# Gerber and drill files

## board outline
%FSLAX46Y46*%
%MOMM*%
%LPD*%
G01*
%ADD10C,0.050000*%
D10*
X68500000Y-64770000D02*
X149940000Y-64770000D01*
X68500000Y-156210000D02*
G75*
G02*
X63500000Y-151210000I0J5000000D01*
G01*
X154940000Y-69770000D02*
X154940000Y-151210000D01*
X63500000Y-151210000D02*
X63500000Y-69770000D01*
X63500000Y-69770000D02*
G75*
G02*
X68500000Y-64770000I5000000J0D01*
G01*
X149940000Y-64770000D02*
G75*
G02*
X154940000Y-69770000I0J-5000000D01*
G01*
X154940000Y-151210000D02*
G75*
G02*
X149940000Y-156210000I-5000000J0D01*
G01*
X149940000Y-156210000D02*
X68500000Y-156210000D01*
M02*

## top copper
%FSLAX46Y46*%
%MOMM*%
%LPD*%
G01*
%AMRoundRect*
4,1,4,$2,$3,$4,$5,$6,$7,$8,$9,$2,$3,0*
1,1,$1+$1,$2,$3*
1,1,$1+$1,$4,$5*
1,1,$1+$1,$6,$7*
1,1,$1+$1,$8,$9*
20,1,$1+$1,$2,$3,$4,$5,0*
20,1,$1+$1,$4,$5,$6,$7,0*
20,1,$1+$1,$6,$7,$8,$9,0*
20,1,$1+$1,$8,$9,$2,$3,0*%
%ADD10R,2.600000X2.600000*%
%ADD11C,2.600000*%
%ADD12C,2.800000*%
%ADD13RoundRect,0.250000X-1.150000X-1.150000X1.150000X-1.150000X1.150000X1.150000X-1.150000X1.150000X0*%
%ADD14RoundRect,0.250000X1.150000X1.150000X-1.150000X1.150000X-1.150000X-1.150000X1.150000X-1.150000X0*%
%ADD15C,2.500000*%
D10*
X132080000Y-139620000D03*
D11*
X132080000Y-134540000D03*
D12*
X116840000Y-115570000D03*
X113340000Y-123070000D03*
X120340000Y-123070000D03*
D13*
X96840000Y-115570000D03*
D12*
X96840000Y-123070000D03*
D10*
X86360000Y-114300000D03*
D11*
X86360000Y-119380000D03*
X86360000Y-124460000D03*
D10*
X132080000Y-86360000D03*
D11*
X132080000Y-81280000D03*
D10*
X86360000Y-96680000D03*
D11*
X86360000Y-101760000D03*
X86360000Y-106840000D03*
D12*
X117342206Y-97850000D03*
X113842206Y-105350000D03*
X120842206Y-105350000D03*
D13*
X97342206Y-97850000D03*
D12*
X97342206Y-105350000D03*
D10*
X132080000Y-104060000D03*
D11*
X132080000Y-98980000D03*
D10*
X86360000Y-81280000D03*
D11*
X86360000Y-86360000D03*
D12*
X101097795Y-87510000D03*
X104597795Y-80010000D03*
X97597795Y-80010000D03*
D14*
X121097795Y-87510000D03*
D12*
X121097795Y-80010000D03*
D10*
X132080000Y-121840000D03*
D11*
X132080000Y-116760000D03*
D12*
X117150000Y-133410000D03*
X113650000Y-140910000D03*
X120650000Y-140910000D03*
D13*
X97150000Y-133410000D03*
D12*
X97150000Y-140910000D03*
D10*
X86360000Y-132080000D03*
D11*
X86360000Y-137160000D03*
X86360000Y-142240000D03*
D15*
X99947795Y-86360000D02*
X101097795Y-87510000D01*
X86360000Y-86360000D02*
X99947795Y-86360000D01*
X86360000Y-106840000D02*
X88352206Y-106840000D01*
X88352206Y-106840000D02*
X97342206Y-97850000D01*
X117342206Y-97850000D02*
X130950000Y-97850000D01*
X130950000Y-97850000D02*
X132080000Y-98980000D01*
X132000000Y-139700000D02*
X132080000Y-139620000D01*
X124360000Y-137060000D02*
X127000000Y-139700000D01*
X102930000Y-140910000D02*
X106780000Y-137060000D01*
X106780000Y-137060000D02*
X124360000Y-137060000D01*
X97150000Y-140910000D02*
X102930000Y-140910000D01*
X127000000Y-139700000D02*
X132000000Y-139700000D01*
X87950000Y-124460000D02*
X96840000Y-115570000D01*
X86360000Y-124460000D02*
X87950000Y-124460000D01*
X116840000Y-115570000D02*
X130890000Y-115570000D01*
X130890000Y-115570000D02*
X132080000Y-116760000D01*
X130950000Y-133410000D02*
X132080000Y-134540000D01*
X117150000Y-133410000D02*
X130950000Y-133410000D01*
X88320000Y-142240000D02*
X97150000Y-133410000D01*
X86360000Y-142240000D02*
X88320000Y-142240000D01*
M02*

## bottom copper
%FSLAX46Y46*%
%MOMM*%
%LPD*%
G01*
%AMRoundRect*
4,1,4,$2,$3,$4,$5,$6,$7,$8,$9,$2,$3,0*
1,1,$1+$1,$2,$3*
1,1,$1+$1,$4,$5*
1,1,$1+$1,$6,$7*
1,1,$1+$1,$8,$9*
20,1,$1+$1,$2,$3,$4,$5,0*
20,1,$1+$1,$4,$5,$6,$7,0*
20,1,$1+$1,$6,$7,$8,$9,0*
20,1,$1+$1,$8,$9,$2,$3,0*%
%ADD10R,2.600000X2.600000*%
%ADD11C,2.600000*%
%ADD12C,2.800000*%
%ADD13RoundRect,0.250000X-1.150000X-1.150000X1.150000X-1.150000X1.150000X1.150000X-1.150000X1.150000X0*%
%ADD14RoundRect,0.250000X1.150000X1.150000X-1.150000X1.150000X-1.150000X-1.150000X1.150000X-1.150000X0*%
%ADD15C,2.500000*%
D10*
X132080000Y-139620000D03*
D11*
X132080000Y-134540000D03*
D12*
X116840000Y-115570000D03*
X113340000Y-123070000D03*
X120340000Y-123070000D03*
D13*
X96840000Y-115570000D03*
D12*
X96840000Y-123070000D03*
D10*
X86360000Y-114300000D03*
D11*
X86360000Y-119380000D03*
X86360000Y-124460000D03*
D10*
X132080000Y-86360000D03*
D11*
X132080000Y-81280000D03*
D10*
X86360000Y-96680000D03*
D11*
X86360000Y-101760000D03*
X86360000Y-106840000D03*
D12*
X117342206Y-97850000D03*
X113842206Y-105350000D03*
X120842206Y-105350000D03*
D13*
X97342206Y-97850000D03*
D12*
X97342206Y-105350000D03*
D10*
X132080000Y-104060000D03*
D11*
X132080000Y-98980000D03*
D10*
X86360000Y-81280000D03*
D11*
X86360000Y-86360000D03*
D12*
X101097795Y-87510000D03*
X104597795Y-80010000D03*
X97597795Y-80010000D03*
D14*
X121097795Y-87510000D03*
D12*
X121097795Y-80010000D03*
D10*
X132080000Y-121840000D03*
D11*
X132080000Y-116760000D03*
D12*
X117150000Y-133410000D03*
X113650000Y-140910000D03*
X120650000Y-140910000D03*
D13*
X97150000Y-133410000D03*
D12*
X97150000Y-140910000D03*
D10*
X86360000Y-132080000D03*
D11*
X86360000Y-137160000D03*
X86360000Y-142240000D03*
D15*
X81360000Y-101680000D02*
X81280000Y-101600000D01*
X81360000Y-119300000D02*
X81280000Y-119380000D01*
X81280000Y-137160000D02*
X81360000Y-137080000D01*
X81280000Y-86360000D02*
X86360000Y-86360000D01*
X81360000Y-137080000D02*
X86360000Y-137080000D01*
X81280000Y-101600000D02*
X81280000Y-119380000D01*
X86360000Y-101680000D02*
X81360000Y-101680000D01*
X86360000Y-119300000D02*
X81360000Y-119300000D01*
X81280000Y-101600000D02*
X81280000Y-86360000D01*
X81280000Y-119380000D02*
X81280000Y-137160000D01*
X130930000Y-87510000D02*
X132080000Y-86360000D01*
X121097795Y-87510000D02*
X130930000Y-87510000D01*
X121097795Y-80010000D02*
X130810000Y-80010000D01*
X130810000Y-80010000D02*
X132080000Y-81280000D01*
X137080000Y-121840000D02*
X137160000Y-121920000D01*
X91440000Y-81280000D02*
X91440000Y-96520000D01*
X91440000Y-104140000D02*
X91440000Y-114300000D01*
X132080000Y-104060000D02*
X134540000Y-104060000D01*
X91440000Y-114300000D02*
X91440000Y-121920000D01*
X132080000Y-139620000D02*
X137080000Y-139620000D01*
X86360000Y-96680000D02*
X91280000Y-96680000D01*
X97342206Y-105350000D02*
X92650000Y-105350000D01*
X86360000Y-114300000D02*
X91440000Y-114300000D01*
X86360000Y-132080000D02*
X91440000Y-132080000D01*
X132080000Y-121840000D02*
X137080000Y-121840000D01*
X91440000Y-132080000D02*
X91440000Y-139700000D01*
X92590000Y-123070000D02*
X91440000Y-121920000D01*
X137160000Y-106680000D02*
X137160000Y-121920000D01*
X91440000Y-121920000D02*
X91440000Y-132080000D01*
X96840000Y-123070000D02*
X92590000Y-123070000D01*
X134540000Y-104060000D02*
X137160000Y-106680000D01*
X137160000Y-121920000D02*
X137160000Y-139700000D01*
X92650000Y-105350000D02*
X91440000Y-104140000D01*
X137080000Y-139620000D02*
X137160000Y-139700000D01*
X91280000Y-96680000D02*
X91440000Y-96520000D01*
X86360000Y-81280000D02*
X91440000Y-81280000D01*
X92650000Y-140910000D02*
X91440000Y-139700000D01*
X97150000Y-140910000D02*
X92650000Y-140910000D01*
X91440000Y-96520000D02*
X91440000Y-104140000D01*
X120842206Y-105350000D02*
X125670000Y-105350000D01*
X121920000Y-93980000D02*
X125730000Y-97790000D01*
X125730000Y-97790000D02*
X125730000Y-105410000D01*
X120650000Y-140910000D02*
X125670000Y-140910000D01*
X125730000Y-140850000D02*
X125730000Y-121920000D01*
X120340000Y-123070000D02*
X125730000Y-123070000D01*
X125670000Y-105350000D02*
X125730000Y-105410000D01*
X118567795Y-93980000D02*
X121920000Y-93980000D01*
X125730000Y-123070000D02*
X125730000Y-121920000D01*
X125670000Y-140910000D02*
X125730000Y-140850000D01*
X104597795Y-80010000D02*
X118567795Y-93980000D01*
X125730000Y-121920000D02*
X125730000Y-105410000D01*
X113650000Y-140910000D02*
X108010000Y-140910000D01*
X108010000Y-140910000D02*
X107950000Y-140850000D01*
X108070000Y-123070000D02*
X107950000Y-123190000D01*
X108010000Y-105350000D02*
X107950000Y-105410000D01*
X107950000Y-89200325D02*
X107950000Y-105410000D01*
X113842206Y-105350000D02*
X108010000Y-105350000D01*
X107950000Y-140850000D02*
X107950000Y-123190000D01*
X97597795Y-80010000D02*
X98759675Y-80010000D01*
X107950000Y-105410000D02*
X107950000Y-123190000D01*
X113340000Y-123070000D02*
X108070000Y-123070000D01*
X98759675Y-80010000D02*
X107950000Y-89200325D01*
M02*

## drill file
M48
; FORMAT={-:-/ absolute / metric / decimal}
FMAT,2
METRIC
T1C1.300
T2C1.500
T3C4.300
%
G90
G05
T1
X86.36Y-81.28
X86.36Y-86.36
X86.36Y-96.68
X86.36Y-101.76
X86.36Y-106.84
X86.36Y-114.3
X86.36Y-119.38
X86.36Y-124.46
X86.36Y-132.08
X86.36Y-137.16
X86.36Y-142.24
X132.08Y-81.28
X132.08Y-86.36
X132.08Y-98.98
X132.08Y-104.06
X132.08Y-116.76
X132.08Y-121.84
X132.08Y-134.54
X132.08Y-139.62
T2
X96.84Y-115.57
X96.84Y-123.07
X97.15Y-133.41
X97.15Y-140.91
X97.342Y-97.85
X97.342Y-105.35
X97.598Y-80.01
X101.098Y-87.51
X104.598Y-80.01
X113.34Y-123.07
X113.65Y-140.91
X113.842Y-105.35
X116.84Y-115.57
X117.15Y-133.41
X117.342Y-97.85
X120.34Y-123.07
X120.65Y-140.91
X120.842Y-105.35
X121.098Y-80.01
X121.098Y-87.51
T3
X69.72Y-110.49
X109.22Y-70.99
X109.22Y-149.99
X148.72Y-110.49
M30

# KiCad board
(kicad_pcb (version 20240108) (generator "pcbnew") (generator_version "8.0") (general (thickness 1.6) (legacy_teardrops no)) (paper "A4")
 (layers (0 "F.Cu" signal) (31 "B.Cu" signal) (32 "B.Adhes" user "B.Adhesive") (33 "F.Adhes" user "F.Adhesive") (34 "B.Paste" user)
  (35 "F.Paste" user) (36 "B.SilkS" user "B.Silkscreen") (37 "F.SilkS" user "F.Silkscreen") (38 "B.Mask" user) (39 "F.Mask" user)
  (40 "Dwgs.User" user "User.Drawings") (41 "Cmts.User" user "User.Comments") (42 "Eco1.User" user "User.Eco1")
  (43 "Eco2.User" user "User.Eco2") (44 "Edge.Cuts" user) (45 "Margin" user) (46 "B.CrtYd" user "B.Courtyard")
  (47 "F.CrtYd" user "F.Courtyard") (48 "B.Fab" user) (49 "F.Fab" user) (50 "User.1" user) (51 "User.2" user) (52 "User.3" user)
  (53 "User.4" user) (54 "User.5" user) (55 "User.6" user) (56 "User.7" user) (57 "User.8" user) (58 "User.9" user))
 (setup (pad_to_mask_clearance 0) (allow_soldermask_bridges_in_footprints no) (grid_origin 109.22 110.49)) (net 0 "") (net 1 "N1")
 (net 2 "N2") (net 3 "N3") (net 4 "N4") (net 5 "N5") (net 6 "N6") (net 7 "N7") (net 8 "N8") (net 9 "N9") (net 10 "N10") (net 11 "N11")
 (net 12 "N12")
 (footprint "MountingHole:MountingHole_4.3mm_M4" (layer "F.Cu") (at 109.22 149.99)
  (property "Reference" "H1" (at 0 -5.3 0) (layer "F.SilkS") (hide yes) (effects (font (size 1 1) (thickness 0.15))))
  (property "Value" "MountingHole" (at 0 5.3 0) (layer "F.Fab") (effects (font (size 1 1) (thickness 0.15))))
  (pad "" np_thru_hole circle (at 0 0) (size 4.3 4.3) (drill 4.3) (layers "*.Cu" "*.Mask")))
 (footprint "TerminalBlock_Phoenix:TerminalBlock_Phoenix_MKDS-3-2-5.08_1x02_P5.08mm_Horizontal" (layer "F.Cu") (at 132.08 139.62 90)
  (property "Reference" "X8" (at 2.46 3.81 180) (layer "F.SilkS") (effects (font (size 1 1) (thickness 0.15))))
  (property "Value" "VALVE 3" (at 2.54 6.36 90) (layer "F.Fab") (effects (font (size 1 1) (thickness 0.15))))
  (pad "1" thru_hole rect (at 0 0 90) (size 2.6 2.6) (drill 1.3) (layers "*.Cu" "*.Mask") (remove_unused_layers no) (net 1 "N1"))
  (pad "2" thru_hole circle (at 5.08 0 90) (size 2.6 2.6) (drill 1.3) (layers "*.Cu" "*.Mask") (remove_unused_layers no) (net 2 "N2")))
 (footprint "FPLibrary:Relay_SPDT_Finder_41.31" (layer "F.Cu") (at 96.84 115.57)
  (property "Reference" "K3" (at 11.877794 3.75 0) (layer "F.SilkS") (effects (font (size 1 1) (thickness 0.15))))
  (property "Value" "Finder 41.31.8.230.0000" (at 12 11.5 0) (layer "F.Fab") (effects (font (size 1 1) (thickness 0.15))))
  (pad "11" thru_hole circle (at 20 0) (size 2.8 2.8) (drill 1.5) (layers "*.Cu" "*.Mask") (remove_unused_layers no) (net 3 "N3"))
  (pad "12" thru_hole circle (at 16.5 7.5) (size 2.8 2.8) (drill 1.5) (layers "*.Cu" "*.Mask") (remove_unused_layers no) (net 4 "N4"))
  (pad "14" thru_hole circle (at 23.5 7.5) (size 2.8 2.8) (drill 1.5) (layers "*.Cu" "*.Mask") (remove_unused_layers no) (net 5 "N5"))
  (pad "A1" thru_hole roundrect (at 0 0) (size 2.8 2.8) (drill 1.5) (layers "*.Cu" "*.Mask") (remove_unused_layers no)
   (roundrect_rratio 0.08928571429) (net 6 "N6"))
  (pad "A2" thru_hole circle (at 0 7.5) (size 2.8 2.8) (drill 1.5) (layers "*.Cu" "*.Mask") (remove_unused_layers no) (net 1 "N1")))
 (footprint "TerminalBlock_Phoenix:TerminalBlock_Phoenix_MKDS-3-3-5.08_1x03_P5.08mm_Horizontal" (layer "F.Cu") (at 86.36 114.3 -90)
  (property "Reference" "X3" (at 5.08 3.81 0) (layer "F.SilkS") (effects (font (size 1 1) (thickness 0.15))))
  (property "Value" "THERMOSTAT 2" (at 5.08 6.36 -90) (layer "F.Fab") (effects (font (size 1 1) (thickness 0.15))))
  (pad "1" thru_hole rect (at 0 0 270) (size 2.6 2.6) (drill 1.3) (layers "*.Cu" "*.Mask") (remove_unused_layers no) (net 1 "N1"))
  (pad "2" thru_hole circle (at 5.08 0 270) (size 2.6 2.6) (drill 1.3) (layers "*.Cu" "*.Mask") (remove_unused_layers no) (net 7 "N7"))
  (pad "3" thru_hole circle (at 10.16 0 270) (size 2.6 2.6) (drill 1.3) (layers "*.Cu" "*.Mask") (remove_unused_layers no) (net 6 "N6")))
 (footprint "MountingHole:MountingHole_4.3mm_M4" (layer "F.Cu") (at 69.72 110.49)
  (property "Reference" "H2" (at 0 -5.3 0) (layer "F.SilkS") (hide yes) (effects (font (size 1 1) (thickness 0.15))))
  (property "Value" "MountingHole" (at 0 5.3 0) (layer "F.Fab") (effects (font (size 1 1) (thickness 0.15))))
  (pad "" np_thru_hole circle (at 0 0) (size 4.3 4.3) (drill 4.3) (layers "*.Cu" "*.Mask")))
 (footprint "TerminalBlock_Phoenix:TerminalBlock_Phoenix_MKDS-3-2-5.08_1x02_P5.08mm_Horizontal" (layer "F.Cu") (at 132.08 86.36 90)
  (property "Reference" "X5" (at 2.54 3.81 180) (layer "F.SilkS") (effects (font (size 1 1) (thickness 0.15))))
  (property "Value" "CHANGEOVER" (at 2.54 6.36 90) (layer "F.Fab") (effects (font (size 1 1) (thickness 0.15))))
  (pad "1" thru_hole rect (at 0 0 90) (size 2.6 2.6) (drill 1.3) (layers "*.Cu" "*.Mask") (remove_unused_layers no) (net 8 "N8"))
  (pad "2" thru_hole circle (at 5.08 0 90) (size 2.6 2.6) (drill 1.3) (layers "*.Cu" "*.Mask") (remove_unused_layers no) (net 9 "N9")))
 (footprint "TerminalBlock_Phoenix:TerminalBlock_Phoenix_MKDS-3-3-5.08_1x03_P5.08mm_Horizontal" (layer "F.Cu") (at 86.36 96.68 -90)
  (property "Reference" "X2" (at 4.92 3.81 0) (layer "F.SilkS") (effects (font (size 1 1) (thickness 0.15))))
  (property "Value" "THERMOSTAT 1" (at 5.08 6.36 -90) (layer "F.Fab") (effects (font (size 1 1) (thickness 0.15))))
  (pad "1" thru_hole rect (at 0 0 270) (size 2.6 2.6) (drill 1.3) (layers "*.Cu" "*.Mask") (remove_unused_layers no) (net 1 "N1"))
  (pad "2" thru_hole circle (at 5.08 0 270) (size 2.6 2.6) (drill 1.3) (layers "*.Cu" "*.Mask") (remove_unused_layers no) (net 7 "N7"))
  (pad "3" thru_hole circle (at 10.16 0 270) (size 2.6 2.6) (drill 1.3) (layers "*.Cu" "*.Mask") (remove_unused_layers no) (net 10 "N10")))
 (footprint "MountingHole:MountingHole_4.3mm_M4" (layer "F.Cu") (at 109.22 70.99)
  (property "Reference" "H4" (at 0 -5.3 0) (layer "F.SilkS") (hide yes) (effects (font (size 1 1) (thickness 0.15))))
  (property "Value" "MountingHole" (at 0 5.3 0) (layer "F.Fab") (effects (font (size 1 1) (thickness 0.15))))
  (pad "" np_thru_hole circle (at 0 0) (size 4.3 4.3) (drill 4.3) (layers "*.Cu" "*.Mask")))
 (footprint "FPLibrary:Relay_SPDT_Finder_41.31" (layer "F.Cu") (at 97.342206 97.85)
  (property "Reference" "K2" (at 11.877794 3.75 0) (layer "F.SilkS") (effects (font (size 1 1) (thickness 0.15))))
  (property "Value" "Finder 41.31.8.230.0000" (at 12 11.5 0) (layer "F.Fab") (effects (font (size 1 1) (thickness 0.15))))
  (pad "11" thru_hole circle (at 20 0) (size 2.8 2.8) (drill 1.5) (layers "*.Cu" "*.Mask") (remove_unused_layers no) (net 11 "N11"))
  (pad "12" thru_hole circle (at 16.5 7.5) (size 2.8 2.8) (drill 1.5) (layers "*.Cu" "*.Mask") (remove_unused_layers no) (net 4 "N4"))
  (pad "14" thru_hole circle (at 23.5 7.5) (size 2.8 2.8) (drill 1.5) (layers "*.Cu" "*.Mask") (remove_unused_layers no) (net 5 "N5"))
  (pad "A1" thru_hole roundrect (at 0 0) (size 2.8 2.8) (drill 1.5) (layers "*.Cu" "*.Mask") (remove_unused_layers no)
   (roundrect_rratio 0.08928571429) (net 10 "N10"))
  (pad "A2" thru_hole circle (at 0 7.5) (size 2.8 2.8) (drill 1.5) (layers "*.Cu" "*.Mask") (remove_unused_layers no) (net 1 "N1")))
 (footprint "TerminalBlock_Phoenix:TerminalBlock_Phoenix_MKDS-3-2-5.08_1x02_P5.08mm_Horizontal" (layer "F.Cu") (at 132.08 104.06 90)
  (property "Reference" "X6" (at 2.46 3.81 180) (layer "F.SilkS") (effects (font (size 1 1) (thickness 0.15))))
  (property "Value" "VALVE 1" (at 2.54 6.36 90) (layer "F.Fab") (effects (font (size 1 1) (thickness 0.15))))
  (pad "1" thru_hole rect (at 0 0 90) (size 2.6 2.6) (drill 1.3) (layers "*.Cu" "*.Mask") (remove_unused_layers no) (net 1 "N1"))
  (pad "2" thru_hole circle (at 5.08 0 90) (size 2.6 2.6) (drill 1.3) (layers "*.Cu" "*.Mask") (remove_unused_layers no) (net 11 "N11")))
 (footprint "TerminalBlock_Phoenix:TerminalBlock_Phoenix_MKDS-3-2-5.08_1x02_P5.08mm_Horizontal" (layer "F.Cu") (at 86.36 81.28 -90)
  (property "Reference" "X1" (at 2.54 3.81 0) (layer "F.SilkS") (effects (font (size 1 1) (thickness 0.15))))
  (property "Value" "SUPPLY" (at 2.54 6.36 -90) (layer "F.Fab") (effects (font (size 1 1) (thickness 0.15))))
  (pad "1" thru_hole rect (at 0 0 270) (size 2.6 2.6) (drill 1.3) (layers "*.Cu" "*.Mask") (remove_unused_layers no) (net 1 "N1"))
  (pad "2" thru_hole circle (at 5.08 0 270) (size 2.6 2.6) (drill 1.3) (layers "*.Cu" "*.Mask") (remove_unused_layers no) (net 7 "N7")))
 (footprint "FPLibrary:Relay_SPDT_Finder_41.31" (layer "F.Cu") (at 121.097795 87.51 180)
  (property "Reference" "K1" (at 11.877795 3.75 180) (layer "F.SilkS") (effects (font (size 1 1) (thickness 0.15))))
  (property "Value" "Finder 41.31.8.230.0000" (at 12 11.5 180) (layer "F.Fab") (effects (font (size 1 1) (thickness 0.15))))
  (pad "11" thru_hole circle (at 20 0 180) (size 2.8 2.8) (drill 1.5) (layers "*.Cu" "*.Mask") (remove_unused_layers no) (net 7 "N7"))
  (pad "12" thru_hole circle (at 16.5 7.5 180) (size 2.8 2.8) (drill 1.5) (layers "*.Cu" "*.Mask") (remove_unused_layers no) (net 5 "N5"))
  (pad "14" thru_hole circle (at 23.5 7.5 180) (size 2.8 2.8) (drill 1.5) (layers "*.Cu" "*.Mask") (remove_unused_layers no) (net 4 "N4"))
  (pad "A1" thru_hole roundrect (at 0 0 180) (size 2.8 2.8) (drill 1.5) (layers "*.Cu" "*.Mask") (remove_unused_layers no)
   (roundrect_rratio 0.08928571429) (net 8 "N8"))
  (pad "A2" thru_hole circle (at 0 7.5 180) (size 2.8 2.8) (drill 1.5) (layers "*.Cu" "*.Mask") (remove_unused_layers no) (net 9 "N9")))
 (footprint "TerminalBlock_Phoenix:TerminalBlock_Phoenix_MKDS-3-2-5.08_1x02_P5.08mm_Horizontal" (layer "F.Cu") (at 132.08 121.84 90)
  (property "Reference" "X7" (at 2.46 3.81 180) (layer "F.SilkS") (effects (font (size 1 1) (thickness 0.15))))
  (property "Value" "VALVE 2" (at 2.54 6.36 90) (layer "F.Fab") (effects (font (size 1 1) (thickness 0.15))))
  (pad "1" thru_hole rect (at 0 0 90) (size 2.6 2.6) (drill 1.3) (layers "*.Cu" "*.Mask") (remove_unused_layers no) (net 1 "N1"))
  (pad "2" thru_hole circle (at 5.08 0 90) (size 2.6 2.6) (drill 1.3) (layers "*.Cu" "*.Mask") (remove_unused_layers no) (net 3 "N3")))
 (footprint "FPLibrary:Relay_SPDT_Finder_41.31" (layer "F.Cu") (at 97.15 133.41)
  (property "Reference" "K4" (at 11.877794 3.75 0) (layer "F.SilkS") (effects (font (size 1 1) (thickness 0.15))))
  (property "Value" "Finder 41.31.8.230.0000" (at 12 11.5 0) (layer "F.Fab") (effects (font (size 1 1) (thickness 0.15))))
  (pad "11" thru_hole circle (at 20 0) (size 2.8 2.8) (drill 1.5) (layers "*.Cu" "*.Mask") (remove_unused_layers no) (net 2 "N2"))
  (pad "12" thru_hole circle (at 16.5 7.5) (size 2.8 2.8) (drill 1.5) (layers "*.Cu" "*.Mask") (remove_unused_layers no) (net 4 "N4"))
  (pad "14" thru_hole circle (at 23.5 7.5) (size 2.8 2.8) (drill 1.5) (layers "*.Cu" "*.Mask") (remove_unused_layers no) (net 5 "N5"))
  (pad "A1" thru_hole roundrect (at 0 0) (size 2.8 2.8) (drill 1.5) (layers "*.Cu" "*.Mask") (remove_unused_layers no)
   (roundrect_rratio 0.08928571429) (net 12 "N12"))
  (pad "A2" thru_hole circle (at 0 7.5) (size 2.8 2.8) (drill 1.5) (layers "*.Cu" "*.Mask") (remove_unused_layers no) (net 1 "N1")))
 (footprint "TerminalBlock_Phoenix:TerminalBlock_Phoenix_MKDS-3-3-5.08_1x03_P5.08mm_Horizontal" (layer "F.Cu") (at 86.36 132.08 -90)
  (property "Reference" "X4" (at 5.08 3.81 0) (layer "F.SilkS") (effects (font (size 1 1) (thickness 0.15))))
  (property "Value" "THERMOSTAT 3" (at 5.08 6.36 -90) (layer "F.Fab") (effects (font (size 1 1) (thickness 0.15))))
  (pad "1" thru_hole rect (at 0 0 270) (size 2.6 2.6) (drill 1.3) (layers "*.Cu" "*.Mask") (remove_unused_layers no) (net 1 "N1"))
  (pad "2" thru_hole circle (at 5.08 0 270) (size 2.6 2.6) (drill 1.3) (layers "*.Cu" "*.Mask") (remove_unused_layers no) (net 7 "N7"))
  (pad "3" thru_hole circle (at 10.16 0 270) (size 2.6 2.6) (drill 1.3) (layers "*.Cu" "*.Mask") (remove_unused_layers no) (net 12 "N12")))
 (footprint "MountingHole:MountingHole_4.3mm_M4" (layer "F.Cu") (at 148.72 110.49)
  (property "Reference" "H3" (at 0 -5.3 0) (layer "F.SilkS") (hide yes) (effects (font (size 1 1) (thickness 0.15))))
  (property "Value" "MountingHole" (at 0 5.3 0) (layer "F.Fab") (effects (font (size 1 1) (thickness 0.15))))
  (pad "" np_thru_hole circle (at 0 0) (size 4.3 4.3) (drill 4.3) (layers "*.Cu" "*.Mask")))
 (gr_line (start 68.5 64.77) (end 149.94 64.77) (stroke (width 0.05) (type default)) (layer "Edge.Cuts"))
 (gr_arc (start 68.5 156.21) (mid 64.964466 154.745534) (end 63.5 151.21) (stroke (width 0.05) (type default)) (layer "Edge.Cuts"))
 (gr_line (start 154.94 69.77) (end 154.94 151.21) (stroke (width 0.05) (type default)) (layer "Edge.Cuts"))
 (gr_line (start 63.5 151.21) (end 63.5 69.77) (stroke (width 0.05) (type default)) (layer "Edge.Cuts"))
 (gr_arc (start 63.5 69.77) (mid 64.964466 66.234466) (end 68.5 64.77) (stroke (width 0.05) (type default)) (layer "Edge.Cuts"))
 (gr_arc (start 149.94 64.77) (mid 153.475534 66.234466) (end 154.94 69.77) (stroke (width 0.05) (type default)) (layer "Edge.Cuts"))
 (gr_arc (start 154.94 151.21) (mid 153.475534 154.745534) (end 149.94 156.21) (stroke (width 0.05) (type default)) (layer "Edge.Cuts"))
 (gr_line (start 149.94 156.21) (end 68.5 156.21) (stroke (width 0.05) (type default)) (layer "Edge.Cuts"))
 (segment (start 99.947795 86.36) (end 101.097795 87.51) (width 2.5) (layer "F.Cu") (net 7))
 (segment (start 86.36 86.36) (end 99.947795 86.36) (width 2.5) (layer "F.Cu") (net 7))
 (segment (start 81.36 101.68) (end 81.28 101.6) (width 2.5) (layer "B.Cu") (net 7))
 (segment (start 81.36 119.3) (end 81.28 119.38) (width 2.5) (layer "B.Cu") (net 7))
 (segment (start 81.28 137.16) (end 81.36 137.08) (width 2.5) (layer "B.Cu") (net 7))
 (segment (start 81.28 86.36) (end 86.36 86.36) (width 2.5) (layer "B.Cu") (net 7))
 (segment (start 81.36 137.08) (end 86.36 137.08) (width 2.5) (layer "B.Cu") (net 7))
 (segment (start 81.28 101.6) (end 81.28 119.38) (width 2.5) (layer "B.Cu") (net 7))
 (segment (start 86.36 101.68) (end 81.36 101.68) (width 2.5) (layer "B.Cu") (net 7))
 (segment (start 86.36 119.3) (end 81.36 119.3) (width 2.5) (layer "B.Cu") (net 7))
 (segment (start 81.28 101.6) (end 81.28 86.36) (width 2.5) (layer "B.Cu") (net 7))
 (segment (start 81.28 119.38) (end 81.28 137.16) (width 2.5) (layer "B.Cu") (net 7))
 (segment (start 130.93 87.51) (end 132.08 86.36) (width 2.5) (layer "B.Cu") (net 8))
 (segment (start 121.097795 87.51) (end 130.93 87.51) (width 2.5) (layer "B.Cu") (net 8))
 (segment (start 121.097795 80.01) (end 130.81 80.01) (width 2.5) (layer "B.Cu") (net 9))
 (segment (start 130.81 80.01) (end 132.08 81.28) (width 2.5) (layer "B.Cu") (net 9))
 (segment (start 86.36 106.84) (end 88.352206 106.84) (width 2.5) (layer "F.Cu") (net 10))
 (segment (start 88.352206 106.84) (end 97.342206 97.85) (width 2.5) (layer "F.Cu") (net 10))
 (segment (start 117.342206 97.85) (end 130.95 97.85) (width 2.5) (layer "F.Cu") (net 11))
 (segment (start 130.95 97.85) (end 132.08 98.98) (width 2.5) (layer "F.Cu") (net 11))
 (segment (start 132 139.7) (end 132.08 139.62) (width 2.5) (layer "F.Cu") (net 1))
 (segment (start 124.36 137.06) (end 127 139.7) (width 2.5) (layer "F.Cu") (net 1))
 (segment (start 102.93 140.91) (end 106.78 137.06) (width 2.5) (layer "F.Cu") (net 1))
 (segment (start 106.78 137.06) (end 124.36 137.06) (width 2.5) (layer "F.Cu") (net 1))
 (segment (start 97.15 140.91) (end 102.93 140.91) (width 2.5) (layer "F.Cu") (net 1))
 (segment (start 127 139.7) (end 132 139.7) (width 2.5) (layer "F.Cu") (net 1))
 (segment (start 137.08 121.84) (end 137.16 121.92) (width 2.5) (layer "B.Cu") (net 1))
 (segment (start 91.44 81.28) (end 91.44 96.52) (width 2.5) (layer "B.Cu") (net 1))
 (segment (start 91.44 104.14) (end 91.44 114.3) (width 2.5) (layer "B.Cu") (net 1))
 (segment (start 132.08 104.06) (end 134.54 104.06) (width 2.5) (layer "B.Cu") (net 1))
 (segment (start 91.44 114.3) (end 91.44 121.92) (width 2.5) (layer "B.Cu") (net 1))
 (segment (start 132.08 139.62) (end 137.08 139.62) (width 2.5) (layer "B.Cu") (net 1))
 (segment (start 86.36 96.68) (end 91.28 96.68) (width 2.5) (layer "B.Cu") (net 1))
 (segment (start 97.342206 105.35) (end 92.65 105.35) (width 2.5) (layer "B.Cu") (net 1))
 (segment (start 86.36 114.3) (end 91.44 114.3) (width 2.5) (layer "B.Cu") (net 1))
 (segment (start 86.36 132.08) (end 91.44 132.08) (width 2.5) (layer "B.Cu") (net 1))
 (segment (start 132.08 121.84) (end 137.08 121.84) (width 2.5) (layer "B.Cu") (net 1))
 (segment (start 91.44 132.08) (end 91.44 139.7) (width 2.5) (layer "B.Cu") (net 1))
 (segment (start 92.59 123.07) (end 91.44 121.92) (width 2.5) (layer "B.Cu") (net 1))
 (segment (start 137.16 106.68) (end 137.16 121.92) (width 2.5) (layer "B.Cu") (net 1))
 (segment (start 91.44 121.92) (end 91.44 132.08) (width 2.5) (layer "B.Cu") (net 1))
 (segment (start 96.84 123.07) (end 92.59 123.07) (width 2.5) (layer "B.Cu") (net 1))
 (segment (start 134.54 104.06) (end 137.16 106.68) (width 2.5) (layer "B.Cu") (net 1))
 (segment (start 137.16 121.92) (end 137.16 139.7) (width 2.5) (layer "B.Cu") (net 1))
 (segment (start 92.65 105.35) (end 91.44 104.14) (width 2.5) (layer "B.Cu") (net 1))
 (segment (start 137.08 139.62) (end 137.16 139.7) (width 2.5) (layer "B.Cu") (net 1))
 (segment (start 91.28 96.68) (end 91.44 96.52) (width 2.5) (layer "B.Cu") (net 1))
 (segment (start 86.36 81.28) (end 91.44 81.28) (width 2.5) (layer "B.Cu") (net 1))
 (segment (start 92.65 140.91) (end 91.44 139.7) (width 2.5) (layer "B.Cu") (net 1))
 (segment (start 97.15 140.91) (end 92.65 140.91) (width 2.5) (layer "B.Cu") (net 1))
 (segment (start 91.44 96.52) (end 91.44 104.14) (width 2.5) (layer "B.Cu") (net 1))
 (segment (start 87.95 124.46) (end 96.84 115.57) (width 2.5) (layer "F.Cu") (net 6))
 (segment (start 86.36 124.46) (end 87.95 124.46) (width 2.5) (layer "F.Cu") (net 6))
 (segment (start 116.84 115.57) (end 130.89 115.57) (width 2.5) (layer "F.Cu") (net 3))
 (segment (start 130.89 115.57) (end 132.08 116.76) (width 2.5) (layer "F.Cu") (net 3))
 (segment (start 120.842206 105.35) (end 125.67 105.35) (width 2.5) (layer "B.Cu") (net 5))
 (segment (start 121.92 93.98) (end 125.73 97.79) (width 2.5) (layer "B.Cu") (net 5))
 (segment (start 125.73 97.79) (end 125.73 105.41) (width 2.5) (layer "B.Cu") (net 5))
 (segment (start 120.65 140.91) (end 125.67 140.91) (width 2.5) (layer "B.Cu") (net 5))
 (segment (start 125.73 140.85) (end 125.73 121.92) (width 2.5) (layer "B.Cu") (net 5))
 (segment (start 120.34 123.07) (end 125.73 123.07) (width 2.5) (layer "B.Cu") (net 5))
 (segment (start 125.67 105.35) (end 125.73 105.41) (width 2.5) (layer "B.Cu") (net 5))
 (segment (start 118.567795 93.98) (end 121.92 93.98) (width 2.5) (layer "B.Cu") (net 5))
 (segment (start 125.73 123.07) (end 125.73 121.92) (width 2.5) (layer "B.Cu") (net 5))
 (segment (start 125.67 140.91) (end 125.73 140.85) (width 2.5) (layer "B.Cu") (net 5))
 (segment (start 104.597795 80.01) (end 118.567795 93.98) (width 2.5) (layer "B.Cu") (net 5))
 (segment (start 125.73 121.92) (end 125.73 105.41) (width 2.5) (layer "B.Cu") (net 5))
 (segment (start 113.65 140.91) (end 108.01 140.91) (width 2.5) (layer "B.Cu") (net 4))
 (segment (start 108.01 140.91) (end 107.95 140.85) (width 2.5) (layer "B.Cu") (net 4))
 (segment (start 108.07 123.07) (end 107.95 123.19) (width 2.5) (layer "B.Cu") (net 4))
 (segment (start 108.01 105.35) (end 107.95 105.41) (width 2.5) (layer "B.Cu") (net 4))
 (segment (start 107.95 89.200325) (end 107.95 105.41) (width 2.5) (layer "B.Cu") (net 4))
 (segment (start 113.842206 105.35) (end 108.01 105.35) (width 2.5) (layer "B.Cu") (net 4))
 (segment (start 107.95 140.85) (end 107.95 123.19) (width 2.5) (layer "B.Cu") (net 4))
 (segment (start 97.597795 80.01) (end 98.759675 80.01) (width 2.5) (layer "B.Cu") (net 4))
 (segment (start 107.95 105.41) (end 107.95 123.19) (width 2.5) (layer "B.Cu") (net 4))
 (segment (start 113.34 123.07) (end 108.07 123.07) (width 2.5) (layer "B.Cu") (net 4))
 (segment (start 98.759675 80.01) (end 107.95 89.200325) (width 2.5) (layer "B.Cu") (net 4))
 (segment (start 130.95 133.41) (end 132.08 134.54) (width 2.5) (layer "F.Cu") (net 2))
 (segment (start 117.15 133.41) (end 130.95 133.41) (width 2.5) (layer "F.Cu") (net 2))
 (segment (start 88.32 142.24) (end 97.15 133.41) (width 2.5) (layer "F.Cu") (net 12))
 (segment (start 86.36 142.24) (end 88.32 142.24) (width 2.5) (layer "F.Cu") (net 12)))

